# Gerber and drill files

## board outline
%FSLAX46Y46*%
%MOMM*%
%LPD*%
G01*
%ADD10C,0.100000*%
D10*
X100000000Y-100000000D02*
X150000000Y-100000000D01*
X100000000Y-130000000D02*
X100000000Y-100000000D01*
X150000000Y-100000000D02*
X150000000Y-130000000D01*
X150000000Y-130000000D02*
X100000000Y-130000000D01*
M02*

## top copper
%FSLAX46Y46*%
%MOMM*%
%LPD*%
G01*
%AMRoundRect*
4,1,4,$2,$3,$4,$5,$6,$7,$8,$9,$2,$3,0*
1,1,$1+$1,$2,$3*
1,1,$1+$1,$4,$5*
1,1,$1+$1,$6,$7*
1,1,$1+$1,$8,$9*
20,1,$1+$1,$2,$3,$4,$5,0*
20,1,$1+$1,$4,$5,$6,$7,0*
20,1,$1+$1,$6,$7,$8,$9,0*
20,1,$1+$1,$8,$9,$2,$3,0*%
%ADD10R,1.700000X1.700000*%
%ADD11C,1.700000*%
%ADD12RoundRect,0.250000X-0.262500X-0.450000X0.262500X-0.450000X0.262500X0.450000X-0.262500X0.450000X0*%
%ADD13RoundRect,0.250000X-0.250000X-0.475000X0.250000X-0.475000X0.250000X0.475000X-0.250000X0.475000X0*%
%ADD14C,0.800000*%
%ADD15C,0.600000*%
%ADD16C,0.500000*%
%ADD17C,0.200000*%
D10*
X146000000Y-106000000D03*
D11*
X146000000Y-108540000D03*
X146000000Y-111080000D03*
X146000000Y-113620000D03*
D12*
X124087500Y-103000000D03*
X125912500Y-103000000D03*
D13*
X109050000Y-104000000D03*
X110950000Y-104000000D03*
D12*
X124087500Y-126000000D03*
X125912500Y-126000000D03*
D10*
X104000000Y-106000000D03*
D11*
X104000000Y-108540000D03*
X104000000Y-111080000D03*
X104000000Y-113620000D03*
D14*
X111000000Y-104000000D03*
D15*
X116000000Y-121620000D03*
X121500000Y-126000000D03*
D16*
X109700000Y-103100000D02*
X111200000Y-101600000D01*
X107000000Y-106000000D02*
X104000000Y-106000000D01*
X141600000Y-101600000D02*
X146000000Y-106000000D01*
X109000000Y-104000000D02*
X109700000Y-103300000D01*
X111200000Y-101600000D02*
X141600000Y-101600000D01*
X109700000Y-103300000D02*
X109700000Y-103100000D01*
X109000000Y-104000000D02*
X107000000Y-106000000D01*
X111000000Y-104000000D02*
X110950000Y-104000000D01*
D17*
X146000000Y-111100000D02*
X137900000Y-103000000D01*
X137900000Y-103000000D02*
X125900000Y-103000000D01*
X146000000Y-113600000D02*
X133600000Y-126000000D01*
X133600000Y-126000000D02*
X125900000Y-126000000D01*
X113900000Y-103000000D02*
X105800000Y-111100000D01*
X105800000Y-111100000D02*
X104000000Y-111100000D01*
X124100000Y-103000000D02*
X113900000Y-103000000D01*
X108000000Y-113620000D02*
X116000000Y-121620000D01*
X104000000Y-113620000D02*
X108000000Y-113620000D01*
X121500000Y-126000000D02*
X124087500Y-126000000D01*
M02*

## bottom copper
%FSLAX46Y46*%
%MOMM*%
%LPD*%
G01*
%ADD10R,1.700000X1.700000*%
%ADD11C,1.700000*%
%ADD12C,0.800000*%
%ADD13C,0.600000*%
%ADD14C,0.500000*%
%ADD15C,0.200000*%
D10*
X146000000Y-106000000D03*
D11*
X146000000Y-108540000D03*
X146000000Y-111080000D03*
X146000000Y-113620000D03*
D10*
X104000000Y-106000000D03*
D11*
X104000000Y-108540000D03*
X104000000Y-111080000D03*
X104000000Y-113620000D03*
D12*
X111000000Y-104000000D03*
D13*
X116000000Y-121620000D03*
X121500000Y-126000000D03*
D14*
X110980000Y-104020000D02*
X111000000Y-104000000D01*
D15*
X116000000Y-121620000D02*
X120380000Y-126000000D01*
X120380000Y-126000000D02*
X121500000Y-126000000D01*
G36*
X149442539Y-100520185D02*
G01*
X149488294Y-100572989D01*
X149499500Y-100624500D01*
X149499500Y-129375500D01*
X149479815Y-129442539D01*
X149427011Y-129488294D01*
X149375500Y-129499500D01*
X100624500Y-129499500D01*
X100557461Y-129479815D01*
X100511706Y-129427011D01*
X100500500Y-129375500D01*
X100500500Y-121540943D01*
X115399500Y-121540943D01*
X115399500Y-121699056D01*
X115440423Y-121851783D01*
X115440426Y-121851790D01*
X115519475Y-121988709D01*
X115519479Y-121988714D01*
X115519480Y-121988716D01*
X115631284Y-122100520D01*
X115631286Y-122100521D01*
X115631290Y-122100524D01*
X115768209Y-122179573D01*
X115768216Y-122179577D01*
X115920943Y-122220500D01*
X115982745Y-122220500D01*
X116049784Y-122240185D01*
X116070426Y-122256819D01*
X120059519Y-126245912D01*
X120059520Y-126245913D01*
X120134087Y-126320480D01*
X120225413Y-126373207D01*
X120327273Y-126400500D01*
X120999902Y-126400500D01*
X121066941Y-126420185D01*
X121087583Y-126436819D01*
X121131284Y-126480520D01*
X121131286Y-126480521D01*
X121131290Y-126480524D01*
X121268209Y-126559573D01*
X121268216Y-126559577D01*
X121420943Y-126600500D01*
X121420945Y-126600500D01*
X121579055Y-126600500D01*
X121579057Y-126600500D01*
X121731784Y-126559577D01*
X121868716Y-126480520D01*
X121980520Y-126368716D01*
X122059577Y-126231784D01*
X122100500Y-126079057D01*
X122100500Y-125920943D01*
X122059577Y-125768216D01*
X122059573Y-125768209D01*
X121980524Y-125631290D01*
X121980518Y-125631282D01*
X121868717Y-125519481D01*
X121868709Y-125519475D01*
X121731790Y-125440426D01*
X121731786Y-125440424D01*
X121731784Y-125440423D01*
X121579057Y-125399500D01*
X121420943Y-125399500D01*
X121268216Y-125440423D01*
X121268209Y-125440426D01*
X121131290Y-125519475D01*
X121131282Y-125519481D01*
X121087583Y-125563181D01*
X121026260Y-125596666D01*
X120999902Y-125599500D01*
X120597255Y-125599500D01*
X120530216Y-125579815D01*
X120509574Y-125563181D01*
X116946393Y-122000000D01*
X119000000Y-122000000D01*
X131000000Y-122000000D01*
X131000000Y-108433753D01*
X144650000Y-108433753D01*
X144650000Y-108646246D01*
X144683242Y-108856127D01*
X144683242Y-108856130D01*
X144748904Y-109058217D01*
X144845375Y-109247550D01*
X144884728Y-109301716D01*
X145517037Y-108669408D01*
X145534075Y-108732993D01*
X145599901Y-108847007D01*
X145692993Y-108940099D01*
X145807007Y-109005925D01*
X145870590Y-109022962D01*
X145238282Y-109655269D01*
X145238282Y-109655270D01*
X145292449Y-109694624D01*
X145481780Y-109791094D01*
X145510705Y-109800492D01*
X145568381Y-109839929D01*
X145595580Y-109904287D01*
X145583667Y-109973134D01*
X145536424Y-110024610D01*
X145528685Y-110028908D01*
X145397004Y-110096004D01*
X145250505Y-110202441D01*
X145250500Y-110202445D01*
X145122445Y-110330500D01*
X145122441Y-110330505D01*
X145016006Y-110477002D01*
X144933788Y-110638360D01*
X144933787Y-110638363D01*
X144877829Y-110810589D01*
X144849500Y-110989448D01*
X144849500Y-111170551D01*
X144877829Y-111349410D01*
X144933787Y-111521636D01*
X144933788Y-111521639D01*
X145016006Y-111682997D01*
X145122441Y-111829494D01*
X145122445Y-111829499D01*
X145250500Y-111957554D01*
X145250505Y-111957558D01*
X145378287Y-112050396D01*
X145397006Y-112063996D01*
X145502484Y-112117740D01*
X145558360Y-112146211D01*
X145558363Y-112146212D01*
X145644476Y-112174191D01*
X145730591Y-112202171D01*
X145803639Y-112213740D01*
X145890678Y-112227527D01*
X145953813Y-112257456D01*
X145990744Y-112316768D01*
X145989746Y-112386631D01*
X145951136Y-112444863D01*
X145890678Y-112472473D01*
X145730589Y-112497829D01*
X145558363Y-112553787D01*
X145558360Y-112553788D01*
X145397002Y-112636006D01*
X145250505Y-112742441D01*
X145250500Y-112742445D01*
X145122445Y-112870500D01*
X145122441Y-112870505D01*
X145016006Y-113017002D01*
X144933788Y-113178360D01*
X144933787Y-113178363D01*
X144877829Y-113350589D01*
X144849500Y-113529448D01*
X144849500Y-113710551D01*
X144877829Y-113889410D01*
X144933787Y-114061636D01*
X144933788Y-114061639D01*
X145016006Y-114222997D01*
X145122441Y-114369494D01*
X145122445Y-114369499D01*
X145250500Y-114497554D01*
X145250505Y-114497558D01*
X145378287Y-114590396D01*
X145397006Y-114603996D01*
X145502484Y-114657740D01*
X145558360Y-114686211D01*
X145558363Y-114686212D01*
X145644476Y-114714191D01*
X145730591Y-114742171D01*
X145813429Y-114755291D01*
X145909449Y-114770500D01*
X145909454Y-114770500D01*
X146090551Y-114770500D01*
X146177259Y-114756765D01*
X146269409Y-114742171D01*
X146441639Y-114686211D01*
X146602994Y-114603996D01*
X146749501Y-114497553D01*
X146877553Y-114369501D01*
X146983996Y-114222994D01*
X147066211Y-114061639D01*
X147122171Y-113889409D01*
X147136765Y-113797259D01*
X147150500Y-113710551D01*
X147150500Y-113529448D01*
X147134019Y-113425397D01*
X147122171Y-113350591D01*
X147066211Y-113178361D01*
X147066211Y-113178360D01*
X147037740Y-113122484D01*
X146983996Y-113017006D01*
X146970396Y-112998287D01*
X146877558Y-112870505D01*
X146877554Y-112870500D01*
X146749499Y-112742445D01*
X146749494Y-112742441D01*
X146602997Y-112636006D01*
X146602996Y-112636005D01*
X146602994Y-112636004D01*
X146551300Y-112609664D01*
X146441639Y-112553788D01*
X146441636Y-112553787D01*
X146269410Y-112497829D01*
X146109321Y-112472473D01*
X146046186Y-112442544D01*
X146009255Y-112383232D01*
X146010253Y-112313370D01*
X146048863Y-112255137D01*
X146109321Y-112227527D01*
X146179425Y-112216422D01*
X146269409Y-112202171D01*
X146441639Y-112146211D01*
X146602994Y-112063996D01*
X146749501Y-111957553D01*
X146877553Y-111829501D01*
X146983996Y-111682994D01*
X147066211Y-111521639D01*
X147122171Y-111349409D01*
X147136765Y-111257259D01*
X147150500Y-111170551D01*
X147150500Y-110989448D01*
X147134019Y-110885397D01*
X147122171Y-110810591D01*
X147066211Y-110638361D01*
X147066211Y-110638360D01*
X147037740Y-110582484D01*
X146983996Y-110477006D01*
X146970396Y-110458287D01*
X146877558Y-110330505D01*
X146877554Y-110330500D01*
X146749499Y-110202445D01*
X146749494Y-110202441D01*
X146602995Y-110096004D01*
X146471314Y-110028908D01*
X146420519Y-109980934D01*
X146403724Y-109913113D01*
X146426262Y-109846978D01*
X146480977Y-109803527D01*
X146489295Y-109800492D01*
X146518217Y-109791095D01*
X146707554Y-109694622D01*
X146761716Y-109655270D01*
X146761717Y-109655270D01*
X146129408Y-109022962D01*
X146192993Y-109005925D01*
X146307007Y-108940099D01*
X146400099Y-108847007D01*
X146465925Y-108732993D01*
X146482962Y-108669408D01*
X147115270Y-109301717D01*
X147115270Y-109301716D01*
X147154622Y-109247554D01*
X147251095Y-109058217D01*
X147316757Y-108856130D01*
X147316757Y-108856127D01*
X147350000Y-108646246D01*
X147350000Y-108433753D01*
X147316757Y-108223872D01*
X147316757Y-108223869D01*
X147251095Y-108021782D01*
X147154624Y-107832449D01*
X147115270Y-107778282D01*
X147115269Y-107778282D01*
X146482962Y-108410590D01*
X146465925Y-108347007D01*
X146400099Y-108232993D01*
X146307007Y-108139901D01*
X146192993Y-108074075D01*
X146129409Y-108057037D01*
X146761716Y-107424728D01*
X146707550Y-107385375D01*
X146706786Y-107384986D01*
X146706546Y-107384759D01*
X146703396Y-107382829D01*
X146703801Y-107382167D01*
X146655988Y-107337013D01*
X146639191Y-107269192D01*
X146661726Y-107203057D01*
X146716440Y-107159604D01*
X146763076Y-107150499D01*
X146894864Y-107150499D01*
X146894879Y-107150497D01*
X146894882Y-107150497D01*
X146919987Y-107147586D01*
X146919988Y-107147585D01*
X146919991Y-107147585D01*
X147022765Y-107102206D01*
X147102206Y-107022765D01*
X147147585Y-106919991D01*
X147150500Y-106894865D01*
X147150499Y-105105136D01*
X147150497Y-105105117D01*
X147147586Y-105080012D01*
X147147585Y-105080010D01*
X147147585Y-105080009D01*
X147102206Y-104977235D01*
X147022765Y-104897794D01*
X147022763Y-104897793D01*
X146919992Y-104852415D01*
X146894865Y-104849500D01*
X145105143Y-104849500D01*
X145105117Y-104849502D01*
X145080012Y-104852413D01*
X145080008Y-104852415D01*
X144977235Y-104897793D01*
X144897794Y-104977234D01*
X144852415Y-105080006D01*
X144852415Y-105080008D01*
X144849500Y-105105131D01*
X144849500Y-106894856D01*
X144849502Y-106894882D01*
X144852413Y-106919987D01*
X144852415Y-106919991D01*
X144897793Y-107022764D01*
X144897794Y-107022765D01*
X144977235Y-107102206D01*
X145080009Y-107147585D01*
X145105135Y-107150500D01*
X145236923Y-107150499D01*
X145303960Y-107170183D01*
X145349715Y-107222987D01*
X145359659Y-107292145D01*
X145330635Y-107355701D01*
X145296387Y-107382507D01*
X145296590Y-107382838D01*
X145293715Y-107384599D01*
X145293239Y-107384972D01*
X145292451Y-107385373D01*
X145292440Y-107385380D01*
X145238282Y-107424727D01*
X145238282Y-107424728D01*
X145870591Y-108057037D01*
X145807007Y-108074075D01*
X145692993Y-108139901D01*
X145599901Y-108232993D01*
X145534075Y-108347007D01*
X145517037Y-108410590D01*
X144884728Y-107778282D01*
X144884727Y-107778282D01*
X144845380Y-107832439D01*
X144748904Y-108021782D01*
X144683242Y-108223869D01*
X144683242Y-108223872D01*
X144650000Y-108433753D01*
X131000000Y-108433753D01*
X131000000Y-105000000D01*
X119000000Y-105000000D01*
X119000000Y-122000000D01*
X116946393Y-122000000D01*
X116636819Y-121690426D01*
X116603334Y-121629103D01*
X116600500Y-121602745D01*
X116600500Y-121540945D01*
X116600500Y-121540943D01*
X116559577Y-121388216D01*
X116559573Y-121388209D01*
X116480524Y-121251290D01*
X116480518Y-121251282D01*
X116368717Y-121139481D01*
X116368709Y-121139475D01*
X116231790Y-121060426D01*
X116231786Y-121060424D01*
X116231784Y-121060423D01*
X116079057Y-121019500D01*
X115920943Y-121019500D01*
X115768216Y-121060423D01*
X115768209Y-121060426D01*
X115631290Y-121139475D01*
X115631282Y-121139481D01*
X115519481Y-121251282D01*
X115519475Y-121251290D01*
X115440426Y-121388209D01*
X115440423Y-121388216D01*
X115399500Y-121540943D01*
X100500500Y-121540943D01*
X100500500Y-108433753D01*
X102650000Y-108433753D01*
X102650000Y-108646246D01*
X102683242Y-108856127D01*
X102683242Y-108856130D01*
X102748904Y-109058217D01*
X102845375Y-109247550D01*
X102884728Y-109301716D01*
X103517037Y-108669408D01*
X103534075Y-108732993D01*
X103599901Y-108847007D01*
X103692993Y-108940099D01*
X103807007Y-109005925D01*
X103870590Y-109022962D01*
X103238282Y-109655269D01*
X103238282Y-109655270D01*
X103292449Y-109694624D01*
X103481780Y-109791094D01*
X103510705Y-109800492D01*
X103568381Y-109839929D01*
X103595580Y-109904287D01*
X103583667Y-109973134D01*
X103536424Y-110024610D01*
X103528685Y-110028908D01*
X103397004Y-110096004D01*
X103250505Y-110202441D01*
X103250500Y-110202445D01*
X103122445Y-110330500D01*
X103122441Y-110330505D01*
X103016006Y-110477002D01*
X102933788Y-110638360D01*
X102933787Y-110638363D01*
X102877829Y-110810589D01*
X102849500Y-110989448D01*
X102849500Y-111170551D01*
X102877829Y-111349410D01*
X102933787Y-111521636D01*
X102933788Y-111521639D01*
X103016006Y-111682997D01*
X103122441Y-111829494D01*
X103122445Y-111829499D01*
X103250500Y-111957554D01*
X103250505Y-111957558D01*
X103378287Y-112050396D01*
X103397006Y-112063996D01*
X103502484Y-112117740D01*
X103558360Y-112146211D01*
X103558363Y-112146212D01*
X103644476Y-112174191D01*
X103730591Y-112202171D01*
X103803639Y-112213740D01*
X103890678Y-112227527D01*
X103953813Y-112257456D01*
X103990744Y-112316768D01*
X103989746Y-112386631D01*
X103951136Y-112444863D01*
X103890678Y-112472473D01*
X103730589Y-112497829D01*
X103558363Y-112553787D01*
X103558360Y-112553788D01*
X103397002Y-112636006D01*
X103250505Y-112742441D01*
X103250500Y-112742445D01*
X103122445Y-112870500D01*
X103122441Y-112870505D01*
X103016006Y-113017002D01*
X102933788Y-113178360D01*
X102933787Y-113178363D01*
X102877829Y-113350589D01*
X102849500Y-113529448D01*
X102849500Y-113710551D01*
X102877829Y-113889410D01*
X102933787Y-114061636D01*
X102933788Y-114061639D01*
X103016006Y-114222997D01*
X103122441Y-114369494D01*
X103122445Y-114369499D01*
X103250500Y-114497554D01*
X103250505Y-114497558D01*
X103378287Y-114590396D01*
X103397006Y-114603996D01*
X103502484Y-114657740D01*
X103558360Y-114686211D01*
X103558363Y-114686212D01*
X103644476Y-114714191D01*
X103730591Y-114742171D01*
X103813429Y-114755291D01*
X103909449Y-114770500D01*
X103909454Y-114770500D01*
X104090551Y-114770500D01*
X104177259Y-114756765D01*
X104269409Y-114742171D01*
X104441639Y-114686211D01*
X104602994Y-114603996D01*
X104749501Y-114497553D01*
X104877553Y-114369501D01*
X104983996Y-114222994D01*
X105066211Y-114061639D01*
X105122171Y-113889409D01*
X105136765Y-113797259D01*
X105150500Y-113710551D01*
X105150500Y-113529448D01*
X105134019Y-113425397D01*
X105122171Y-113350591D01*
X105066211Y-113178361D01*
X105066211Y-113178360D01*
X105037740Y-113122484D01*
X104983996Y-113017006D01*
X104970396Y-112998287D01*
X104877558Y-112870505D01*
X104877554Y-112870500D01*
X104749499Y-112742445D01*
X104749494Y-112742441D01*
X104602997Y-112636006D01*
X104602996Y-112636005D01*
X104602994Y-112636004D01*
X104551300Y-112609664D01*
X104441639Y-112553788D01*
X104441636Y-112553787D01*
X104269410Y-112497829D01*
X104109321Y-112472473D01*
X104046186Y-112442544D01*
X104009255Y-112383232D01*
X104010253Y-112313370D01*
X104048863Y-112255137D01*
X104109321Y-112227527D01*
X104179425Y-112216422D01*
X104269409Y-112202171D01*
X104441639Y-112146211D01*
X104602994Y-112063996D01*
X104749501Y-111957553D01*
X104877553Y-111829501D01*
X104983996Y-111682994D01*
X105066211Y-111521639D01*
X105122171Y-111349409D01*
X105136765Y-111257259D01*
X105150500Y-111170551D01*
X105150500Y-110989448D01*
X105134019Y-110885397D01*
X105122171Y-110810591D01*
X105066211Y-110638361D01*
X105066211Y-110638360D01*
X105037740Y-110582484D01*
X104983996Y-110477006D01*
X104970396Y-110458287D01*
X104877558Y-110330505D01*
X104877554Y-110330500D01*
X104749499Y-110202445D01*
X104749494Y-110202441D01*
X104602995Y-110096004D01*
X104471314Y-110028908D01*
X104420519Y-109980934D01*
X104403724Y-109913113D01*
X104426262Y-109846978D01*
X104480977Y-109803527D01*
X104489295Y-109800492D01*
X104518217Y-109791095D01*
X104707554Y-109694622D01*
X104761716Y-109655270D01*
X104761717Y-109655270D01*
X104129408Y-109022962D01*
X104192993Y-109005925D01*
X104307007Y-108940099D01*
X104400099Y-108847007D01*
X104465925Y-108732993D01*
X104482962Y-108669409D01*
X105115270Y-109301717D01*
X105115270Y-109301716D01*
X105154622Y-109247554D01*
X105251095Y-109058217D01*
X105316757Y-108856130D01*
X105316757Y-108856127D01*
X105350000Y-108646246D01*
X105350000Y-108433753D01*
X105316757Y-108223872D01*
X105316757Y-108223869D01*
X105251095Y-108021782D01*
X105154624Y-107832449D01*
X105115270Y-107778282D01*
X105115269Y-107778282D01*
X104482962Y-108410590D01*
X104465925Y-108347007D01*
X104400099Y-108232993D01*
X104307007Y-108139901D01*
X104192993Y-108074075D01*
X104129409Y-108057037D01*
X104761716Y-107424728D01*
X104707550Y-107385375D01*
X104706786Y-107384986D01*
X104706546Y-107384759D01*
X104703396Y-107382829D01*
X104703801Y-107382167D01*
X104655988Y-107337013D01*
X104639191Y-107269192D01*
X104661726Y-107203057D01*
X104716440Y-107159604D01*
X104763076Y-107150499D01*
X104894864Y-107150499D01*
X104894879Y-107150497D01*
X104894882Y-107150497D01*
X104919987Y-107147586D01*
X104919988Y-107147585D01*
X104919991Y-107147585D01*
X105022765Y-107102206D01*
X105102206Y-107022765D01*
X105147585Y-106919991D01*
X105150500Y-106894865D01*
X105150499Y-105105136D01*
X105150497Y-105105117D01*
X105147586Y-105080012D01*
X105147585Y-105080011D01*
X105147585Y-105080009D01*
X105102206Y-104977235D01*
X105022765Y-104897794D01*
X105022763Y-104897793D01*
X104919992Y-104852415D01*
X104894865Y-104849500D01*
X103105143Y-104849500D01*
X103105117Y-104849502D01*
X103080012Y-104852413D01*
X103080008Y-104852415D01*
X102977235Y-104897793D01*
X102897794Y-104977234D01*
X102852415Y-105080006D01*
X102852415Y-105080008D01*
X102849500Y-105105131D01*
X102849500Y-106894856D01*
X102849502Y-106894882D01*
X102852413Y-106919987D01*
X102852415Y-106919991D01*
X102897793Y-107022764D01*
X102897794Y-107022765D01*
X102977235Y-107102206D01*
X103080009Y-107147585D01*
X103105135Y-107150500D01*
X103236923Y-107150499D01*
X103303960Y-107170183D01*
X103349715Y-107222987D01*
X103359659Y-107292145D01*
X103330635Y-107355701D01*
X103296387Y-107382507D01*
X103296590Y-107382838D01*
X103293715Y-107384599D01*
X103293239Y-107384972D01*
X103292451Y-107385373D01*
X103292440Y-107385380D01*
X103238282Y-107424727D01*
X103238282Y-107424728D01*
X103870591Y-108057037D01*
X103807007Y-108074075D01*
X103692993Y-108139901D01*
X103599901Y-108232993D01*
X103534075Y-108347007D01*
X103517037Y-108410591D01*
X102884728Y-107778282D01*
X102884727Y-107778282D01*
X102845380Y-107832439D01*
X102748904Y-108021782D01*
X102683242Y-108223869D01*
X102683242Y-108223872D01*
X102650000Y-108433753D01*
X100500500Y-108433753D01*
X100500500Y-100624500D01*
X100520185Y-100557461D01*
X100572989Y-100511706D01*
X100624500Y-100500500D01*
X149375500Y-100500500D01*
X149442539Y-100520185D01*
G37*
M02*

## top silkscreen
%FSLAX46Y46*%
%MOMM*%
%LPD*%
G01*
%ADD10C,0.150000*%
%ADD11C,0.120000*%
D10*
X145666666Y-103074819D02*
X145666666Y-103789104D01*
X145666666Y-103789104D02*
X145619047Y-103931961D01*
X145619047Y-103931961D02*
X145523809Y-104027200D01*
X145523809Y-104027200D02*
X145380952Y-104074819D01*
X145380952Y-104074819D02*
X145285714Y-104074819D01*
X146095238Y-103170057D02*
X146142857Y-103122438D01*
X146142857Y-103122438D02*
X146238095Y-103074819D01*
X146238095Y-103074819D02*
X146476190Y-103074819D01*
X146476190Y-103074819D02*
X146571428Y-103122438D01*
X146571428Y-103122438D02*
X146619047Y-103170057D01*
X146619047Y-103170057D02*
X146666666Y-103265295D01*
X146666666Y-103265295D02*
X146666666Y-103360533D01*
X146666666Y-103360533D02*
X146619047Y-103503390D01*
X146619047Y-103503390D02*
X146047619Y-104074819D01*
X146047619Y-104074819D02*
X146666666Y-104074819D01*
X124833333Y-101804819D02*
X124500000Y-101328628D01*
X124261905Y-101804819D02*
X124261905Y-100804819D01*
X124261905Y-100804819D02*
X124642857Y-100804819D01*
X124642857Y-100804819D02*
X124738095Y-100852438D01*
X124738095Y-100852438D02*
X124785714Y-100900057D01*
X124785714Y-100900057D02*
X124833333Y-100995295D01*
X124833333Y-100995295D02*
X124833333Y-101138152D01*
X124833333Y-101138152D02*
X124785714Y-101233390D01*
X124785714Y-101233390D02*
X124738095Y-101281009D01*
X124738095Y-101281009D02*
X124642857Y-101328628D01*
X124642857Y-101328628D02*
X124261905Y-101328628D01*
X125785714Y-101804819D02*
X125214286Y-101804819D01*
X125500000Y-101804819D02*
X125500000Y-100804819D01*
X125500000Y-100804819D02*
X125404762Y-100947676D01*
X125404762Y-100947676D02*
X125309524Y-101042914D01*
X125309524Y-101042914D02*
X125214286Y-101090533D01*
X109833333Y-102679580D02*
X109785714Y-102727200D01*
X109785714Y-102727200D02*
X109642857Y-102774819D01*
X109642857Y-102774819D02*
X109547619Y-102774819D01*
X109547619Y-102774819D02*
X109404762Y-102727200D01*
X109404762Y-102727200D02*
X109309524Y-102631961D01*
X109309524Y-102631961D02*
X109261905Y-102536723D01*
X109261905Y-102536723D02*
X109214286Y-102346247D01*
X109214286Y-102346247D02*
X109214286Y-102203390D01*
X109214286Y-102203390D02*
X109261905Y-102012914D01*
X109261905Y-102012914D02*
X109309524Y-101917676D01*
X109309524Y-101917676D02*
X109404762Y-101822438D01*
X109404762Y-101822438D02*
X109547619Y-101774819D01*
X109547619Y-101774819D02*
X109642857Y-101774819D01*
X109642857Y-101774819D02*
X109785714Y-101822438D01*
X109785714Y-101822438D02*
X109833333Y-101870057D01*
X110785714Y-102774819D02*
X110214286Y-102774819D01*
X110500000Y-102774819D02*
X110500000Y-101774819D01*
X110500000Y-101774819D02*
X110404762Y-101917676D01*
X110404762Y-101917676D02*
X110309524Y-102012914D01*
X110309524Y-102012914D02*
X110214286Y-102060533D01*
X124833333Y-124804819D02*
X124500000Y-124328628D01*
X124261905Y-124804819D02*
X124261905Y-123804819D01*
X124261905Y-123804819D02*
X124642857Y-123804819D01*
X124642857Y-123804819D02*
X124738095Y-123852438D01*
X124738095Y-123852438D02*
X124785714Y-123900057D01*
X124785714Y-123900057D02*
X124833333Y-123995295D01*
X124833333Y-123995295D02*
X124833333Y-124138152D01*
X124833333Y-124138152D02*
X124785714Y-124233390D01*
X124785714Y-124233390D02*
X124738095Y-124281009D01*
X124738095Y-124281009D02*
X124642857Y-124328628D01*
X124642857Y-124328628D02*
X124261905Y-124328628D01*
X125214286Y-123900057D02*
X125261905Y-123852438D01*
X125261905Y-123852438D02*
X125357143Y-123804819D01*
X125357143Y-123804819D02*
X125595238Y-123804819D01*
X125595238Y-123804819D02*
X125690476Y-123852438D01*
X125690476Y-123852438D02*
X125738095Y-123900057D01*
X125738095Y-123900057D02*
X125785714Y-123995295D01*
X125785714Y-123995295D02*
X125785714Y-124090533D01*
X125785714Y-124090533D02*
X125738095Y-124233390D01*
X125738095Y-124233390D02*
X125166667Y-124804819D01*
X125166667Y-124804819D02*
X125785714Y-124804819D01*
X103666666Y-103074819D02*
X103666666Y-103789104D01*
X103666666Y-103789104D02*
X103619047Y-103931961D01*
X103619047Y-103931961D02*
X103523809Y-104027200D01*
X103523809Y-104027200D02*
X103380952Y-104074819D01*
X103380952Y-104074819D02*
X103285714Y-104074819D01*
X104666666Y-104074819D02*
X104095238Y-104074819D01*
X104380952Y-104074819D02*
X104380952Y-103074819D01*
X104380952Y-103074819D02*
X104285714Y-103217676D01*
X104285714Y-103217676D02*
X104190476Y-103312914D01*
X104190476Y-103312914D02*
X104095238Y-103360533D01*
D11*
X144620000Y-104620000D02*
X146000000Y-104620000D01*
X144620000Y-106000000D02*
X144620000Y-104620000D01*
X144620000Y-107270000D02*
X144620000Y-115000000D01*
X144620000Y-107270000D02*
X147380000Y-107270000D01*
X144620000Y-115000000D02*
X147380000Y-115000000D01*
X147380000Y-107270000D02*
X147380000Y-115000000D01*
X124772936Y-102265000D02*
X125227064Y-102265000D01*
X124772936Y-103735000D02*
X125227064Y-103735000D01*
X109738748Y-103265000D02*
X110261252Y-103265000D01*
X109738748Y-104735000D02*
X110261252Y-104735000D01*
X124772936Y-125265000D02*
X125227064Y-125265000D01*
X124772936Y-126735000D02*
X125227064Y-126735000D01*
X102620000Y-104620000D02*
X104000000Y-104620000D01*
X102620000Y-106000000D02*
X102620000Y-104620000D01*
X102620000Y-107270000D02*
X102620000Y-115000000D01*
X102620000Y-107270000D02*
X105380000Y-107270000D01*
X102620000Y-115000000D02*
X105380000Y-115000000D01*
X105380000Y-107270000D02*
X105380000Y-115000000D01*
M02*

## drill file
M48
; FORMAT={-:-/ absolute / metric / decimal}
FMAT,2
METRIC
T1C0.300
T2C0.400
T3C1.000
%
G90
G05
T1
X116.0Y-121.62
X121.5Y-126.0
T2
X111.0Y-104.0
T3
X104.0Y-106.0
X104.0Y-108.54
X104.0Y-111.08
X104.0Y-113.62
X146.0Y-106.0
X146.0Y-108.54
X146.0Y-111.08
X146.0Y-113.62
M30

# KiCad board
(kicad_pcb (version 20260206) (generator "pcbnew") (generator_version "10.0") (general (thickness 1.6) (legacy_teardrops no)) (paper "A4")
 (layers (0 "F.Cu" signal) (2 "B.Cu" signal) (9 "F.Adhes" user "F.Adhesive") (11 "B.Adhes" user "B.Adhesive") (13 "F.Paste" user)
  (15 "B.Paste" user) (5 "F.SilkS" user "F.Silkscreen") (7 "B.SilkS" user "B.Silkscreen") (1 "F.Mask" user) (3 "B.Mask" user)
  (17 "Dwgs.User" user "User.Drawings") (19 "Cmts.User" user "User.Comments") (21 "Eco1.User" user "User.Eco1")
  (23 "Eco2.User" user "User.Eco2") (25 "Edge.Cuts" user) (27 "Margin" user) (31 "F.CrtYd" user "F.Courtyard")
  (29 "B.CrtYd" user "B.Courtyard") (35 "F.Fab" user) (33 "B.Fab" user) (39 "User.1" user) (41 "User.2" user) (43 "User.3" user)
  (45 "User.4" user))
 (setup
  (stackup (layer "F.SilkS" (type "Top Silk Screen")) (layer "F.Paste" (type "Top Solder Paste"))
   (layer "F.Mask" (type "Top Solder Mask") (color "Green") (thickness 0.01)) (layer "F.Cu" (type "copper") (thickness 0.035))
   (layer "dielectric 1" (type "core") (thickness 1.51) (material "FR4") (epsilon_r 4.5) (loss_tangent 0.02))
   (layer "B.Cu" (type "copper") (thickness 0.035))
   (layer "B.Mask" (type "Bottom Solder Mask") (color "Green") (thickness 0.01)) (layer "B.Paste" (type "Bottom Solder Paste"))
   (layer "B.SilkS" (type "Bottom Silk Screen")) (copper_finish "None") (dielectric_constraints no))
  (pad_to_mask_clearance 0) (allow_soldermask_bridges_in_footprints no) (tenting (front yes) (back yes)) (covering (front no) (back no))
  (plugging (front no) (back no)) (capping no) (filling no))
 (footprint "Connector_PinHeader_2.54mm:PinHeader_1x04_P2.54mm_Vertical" (layer "F.Cu") (at 146 106)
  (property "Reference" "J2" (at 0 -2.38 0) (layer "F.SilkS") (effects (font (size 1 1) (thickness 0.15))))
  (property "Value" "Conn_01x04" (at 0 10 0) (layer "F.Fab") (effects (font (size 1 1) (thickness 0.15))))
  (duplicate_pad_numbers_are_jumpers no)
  (fp_line (start -1.38 -1.38) (end 0 -1.38) (stroke (width 0.12) (type solid)) (layer "F.SilkS"))
  (fp_line (start -1.38 0) (end -1.38 -1.38) (stroke (width 0.12) (type solid)) (layer "F.SilkS"))
  (fp_line (start -1.38 1.27) (end -1.38 9) (stroke (width 0.12) (type solid)) (layer "F.SilkS"))
  (fp_line (start -1.38 1.27) (end 1.38 1.27) (stroke (width 0.12) (type solid)) (layer "F.SilkS"))
  (fp_line (start -1.38 9) (end 1.38 9) (stroke (width 0.12) (type solid)) (layer "F.SilkS"))
  (fp_line (start 1.38 1.27) (end 1.38 9) (stroke (width 0.12) (type solid)) (layer "F.SilkS"))
  (pad "1" thru_hole rect (at 0 0) (size 1.7 1.7) (drill 1) (layers "*.Cu" "*.Mask") (remove_unused_layers no) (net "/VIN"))
  (pad "2" thru_hole circle (at 0 2.54) (size 1.7 1.7) (drill 1) (layers "*.Cu" "*.Mask") (remove_unused_layers no) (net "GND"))
  (pad "3" thru_hole circle (at 0 5.08) (size 1.7 1.7) (drill 1) (layers "*.Cu" "*.Mask") (remove_unused_layers no) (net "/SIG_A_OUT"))
  (pad "4" thru_hole circle (at 0 7.62) (size 1.7 1.7) (drill 1) (layers "*.Cu" "*.Mask") (remove_unused_layers no) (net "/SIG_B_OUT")))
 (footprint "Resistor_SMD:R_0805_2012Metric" (layer "F.Cu") (at 125 103)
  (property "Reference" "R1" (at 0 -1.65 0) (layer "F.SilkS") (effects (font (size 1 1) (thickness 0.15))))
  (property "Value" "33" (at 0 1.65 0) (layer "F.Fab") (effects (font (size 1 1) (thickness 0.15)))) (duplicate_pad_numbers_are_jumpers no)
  (fp_line (start -0.227064 -0.735) (end 0.227064 -0.735) (stroke (width 0.12) (type solid)) (layer "F.SilkS"))
  (fp_line (start -0.227064 0.735) (end 0.227064 0.735) (stroke (width 0.12) (type solid)) (layer "F.SilkS"))
  (pad "1" smd roundrect (at -0.9125 0) (size 1.025 1.4) (layers "F.Cu" "F.Mask" "F.Paste") (roundrect_rratio 0.243902) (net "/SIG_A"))
  (pad "2" smd roundrect (at 0.9125 0) (size 1.025 1.4) (layers "F.Cu" "F.Mask" "F.Paste") (roundrect_rratio 0.243902) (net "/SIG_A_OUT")))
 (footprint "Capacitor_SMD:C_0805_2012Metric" (layer "F.Cu") (at 110 104)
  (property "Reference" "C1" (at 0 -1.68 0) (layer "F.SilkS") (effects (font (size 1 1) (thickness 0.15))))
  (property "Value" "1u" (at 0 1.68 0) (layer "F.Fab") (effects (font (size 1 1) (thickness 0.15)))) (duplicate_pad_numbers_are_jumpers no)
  (fp_line (start -0.261252 -0.735) (end 0.261252 -0.735) (stroke (width 0.12) (type solid)) (layer "F.SilkS"))
  (fp_line (start -0.261252 0.735) (end 0.261252 0.735) (stroke (width 0.12) (type solid)) (layer "F.SilkS"))
  (pad "1" smd roundrect (at -0.95 0) (size 1 1.45) (layers "F.Cu" "F.Mask" "F.Paste") (roundrect_rratio 0.25) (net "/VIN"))
  (pad "2" smd roundrect (at 0.95 0) (size 1 1.45) (layers "F.Cu" "F.Mask" "F.Paste") (roundrect_rratio 0.25) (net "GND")))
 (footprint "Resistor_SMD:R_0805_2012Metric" (layer "F.Cu") (at 125 126)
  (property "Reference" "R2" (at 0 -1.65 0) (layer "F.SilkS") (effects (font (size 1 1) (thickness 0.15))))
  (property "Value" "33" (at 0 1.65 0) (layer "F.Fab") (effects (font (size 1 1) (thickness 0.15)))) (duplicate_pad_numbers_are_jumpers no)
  (fp_line (start -0.227064 -0.735) (end 0.227064 -0.735) (stroke (width 0.12) (type solid)) (layer "F.SilkS"))
  (fp_line (start -0.227064 0.735) (end 0.227064 0.735) (stroke (width 0.12) (type solid)) (layer "F.SilkS"))
  (pad "1" smd roundrect (at -0.9125 0) (size 1.025 1.4) (layers "F.Cu" "F.Mask" "F.Paste") (roundrect_rratio 0.243902) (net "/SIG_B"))
  (pad "2" smd roundrect (at 0.9125 0) (size 1.025 1.4) (layers "F.Cu" "F.Mask" "F.Paste") (roundrect_rratio 0.243902) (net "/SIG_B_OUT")))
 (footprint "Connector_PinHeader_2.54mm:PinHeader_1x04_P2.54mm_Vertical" (layer "F.Cu") (at 104 106)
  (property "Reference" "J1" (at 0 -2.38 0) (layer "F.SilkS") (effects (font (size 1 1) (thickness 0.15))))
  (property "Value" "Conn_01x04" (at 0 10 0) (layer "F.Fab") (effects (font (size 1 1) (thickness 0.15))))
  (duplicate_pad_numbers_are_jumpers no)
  (fp_line (start -1.38 -1.38) (end 0 -1.38) (stroke (width 0.12) (type solid)) (layer "F.SilkS"))
  (fp_line (start -1.38 0) (end -1.38 -1.38) (stroke (width 0.12) (type solid)) (layer "F.SilkS"))
  (fp_line (start -1.38 1.27) (end -1.38 9) (stroke (width 0.12) (type solid)) (layer "F.SilkS"))
  (fp_line (start -1.38 1.27) (end 1.38 1.27) (stroke (width 0.12) (type solid)) (layer "F.SilkS"))
  (fp_line (start -1.38 9) (end 1.38 9) (stroke (width 0.12) (type solid)) (layer "F.SilkS"))
  (fp_line (start 1.38 1.27) (end 1.38 9) (stroke (width 0.12) (type solid)) (layer "F.SilkS"))
  (pad "1" thru_hole rect (at 0 0) (size 1.7 1.7) (drill 1) (layers "*.Cu" "*.Mask") (remove_unused_layers no) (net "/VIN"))
  (pad "2" thru_hole circle (at 0 2.54) (size 1.7 1.7) (drill 1) (layers "*.Cu" "*.Mask") (remove_unused_layers no) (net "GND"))
  (pad "3" thru_hole circle (at 0 5.08) (size 1.7 1.7) (drill 1) (layers "*.Cu" "*.Mask") (remove_unused_layers no) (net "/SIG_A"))
  (pad "4" thru_hole circle (at 0 7.62) (size 1.7 1.7) (drill 1) (layers "*.Cu" "*.Mask") (remove_unused_layers no) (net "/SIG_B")))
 (gr_line (start 100 100) (end 150 100) (stroke (width 0.1) (type default)) (layer "Edge.Cuts"))
 (gr_line (start 100 130) (end 100 100) (stroke (width 0.1) (type default)) (layer "Edge.Cuts"))
 (gr_line (start 150 100) (end 150 130) (stroke (width 0.1) (type default)) (layer "Edge.Cuts"))
 (gr_line (start 150 130) (end 100 130) (stroke (width 0.1) (type default)) (layer "Edge.Cuts"))
 (segment (start 109.7 103.1) (end 111.2 101.6) (width 0.5) (layer "F.Cu") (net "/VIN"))
 (segment (start 107 106) (end 104 106) (width 0.5) (layer "F.Cu") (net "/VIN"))
 (segment (start 141.6 101.6) (end 146 106) (width 0.5) (layer "F.Cu") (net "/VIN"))
 (segment (start 109 104) (end 109.7 103.3) (width 0.5) (layer "F.Cu") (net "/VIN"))
 (segment (start 111.2 101.6) (end 141.6 101.6) (width 0.5) (layer "F.Cu") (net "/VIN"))
 (segment (start 109.7 103.3) (end 109.7 103.1) (width 0.5) (layer "F.Cu") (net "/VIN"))
 (segment (start 109 104) (end 107 106) (width 0.5) (layer "F.Cu") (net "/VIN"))
 (segment (start 111 104) (end 110.95 104) (width 0.5) (layer "F.Cu") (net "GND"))
 (via (at 111 104) (size 0.8) (drill 0.4) (layers "F.Cu" "B.Cu") (capping yes) (filling yes) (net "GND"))
 (segment (start 110.98 104.02) (end 111 104) (width 0.5) (layer "B.Cu") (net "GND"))
 (segment (start 146 111.1) (end 137.9 103) (width 0.2) (layer "F.Cu") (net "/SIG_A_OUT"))
 (segment (start 137.9 103) (end 125.9 103) (width 0.2) (layer "F.Cu") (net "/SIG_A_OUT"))
 (segment (start 146 113.6) (end 133.6 126) (width 0.2) (layer "F.Cu") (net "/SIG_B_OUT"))
 (segment (start 133.6 126) (end 125.9 126) (width 0.2) (layer "F.Cu") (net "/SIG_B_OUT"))
 (segment (start 113.9 103) (end 105.8 111.1) (width 0.2) (layer "F.Cu") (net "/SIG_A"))
 (segment (start 105.8 111.1) (end 104 111.1) (width 0.2) (layer "F.Cu") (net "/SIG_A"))
 (segment (start 124.1 103) (end 113.9 103) (width 0.2) (layer "F.Cu") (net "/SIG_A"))
 (segment (start 108 113.62) (end 116 121.62) (width 0.2) (locked yes) (layer "F.Cu") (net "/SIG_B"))
 (segment (start 104 113.62) (end 108 113.62) (width 0.2) (locked yes) (layer "F.Cu") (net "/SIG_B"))
 (segment (start 121.5 126) (end 124.0875 126) (width 0.2) (locked yes) (layer "F.Cu") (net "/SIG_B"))
 (via (at 116 121.62) (size 0.6) (drill 0.3) (layers "F.Cu" "B.Cu") (locked yes) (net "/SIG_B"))
 (via (at 121.5 126) (size 0.6) (drill 0.3) (layers "F.Cu" "B.Cu") (locked yes) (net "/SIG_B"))
 (segment (start 116 121.62) (end 120.38 126) (width 0.2) (locked yes) (layer "B.Cu") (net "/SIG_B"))
 (segment (start 120.38 126) (end 121.5 126) (width 0.2) (locked yes) (layer "B.Cu") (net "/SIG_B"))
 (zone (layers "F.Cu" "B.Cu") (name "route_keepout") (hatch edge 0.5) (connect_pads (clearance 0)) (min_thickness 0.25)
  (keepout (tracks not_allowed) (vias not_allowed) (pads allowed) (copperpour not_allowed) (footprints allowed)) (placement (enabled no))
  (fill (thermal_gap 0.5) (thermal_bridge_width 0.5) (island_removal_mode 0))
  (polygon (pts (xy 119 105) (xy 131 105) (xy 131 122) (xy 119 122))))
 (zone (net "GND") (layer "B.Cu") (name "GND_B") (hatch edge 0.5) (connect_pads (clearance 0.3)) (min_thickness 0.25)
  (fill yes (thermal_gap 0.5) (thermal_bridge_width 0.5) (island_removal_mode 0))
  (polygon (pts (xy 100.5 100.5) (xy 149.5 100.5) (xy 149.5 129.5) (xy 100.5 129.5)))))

